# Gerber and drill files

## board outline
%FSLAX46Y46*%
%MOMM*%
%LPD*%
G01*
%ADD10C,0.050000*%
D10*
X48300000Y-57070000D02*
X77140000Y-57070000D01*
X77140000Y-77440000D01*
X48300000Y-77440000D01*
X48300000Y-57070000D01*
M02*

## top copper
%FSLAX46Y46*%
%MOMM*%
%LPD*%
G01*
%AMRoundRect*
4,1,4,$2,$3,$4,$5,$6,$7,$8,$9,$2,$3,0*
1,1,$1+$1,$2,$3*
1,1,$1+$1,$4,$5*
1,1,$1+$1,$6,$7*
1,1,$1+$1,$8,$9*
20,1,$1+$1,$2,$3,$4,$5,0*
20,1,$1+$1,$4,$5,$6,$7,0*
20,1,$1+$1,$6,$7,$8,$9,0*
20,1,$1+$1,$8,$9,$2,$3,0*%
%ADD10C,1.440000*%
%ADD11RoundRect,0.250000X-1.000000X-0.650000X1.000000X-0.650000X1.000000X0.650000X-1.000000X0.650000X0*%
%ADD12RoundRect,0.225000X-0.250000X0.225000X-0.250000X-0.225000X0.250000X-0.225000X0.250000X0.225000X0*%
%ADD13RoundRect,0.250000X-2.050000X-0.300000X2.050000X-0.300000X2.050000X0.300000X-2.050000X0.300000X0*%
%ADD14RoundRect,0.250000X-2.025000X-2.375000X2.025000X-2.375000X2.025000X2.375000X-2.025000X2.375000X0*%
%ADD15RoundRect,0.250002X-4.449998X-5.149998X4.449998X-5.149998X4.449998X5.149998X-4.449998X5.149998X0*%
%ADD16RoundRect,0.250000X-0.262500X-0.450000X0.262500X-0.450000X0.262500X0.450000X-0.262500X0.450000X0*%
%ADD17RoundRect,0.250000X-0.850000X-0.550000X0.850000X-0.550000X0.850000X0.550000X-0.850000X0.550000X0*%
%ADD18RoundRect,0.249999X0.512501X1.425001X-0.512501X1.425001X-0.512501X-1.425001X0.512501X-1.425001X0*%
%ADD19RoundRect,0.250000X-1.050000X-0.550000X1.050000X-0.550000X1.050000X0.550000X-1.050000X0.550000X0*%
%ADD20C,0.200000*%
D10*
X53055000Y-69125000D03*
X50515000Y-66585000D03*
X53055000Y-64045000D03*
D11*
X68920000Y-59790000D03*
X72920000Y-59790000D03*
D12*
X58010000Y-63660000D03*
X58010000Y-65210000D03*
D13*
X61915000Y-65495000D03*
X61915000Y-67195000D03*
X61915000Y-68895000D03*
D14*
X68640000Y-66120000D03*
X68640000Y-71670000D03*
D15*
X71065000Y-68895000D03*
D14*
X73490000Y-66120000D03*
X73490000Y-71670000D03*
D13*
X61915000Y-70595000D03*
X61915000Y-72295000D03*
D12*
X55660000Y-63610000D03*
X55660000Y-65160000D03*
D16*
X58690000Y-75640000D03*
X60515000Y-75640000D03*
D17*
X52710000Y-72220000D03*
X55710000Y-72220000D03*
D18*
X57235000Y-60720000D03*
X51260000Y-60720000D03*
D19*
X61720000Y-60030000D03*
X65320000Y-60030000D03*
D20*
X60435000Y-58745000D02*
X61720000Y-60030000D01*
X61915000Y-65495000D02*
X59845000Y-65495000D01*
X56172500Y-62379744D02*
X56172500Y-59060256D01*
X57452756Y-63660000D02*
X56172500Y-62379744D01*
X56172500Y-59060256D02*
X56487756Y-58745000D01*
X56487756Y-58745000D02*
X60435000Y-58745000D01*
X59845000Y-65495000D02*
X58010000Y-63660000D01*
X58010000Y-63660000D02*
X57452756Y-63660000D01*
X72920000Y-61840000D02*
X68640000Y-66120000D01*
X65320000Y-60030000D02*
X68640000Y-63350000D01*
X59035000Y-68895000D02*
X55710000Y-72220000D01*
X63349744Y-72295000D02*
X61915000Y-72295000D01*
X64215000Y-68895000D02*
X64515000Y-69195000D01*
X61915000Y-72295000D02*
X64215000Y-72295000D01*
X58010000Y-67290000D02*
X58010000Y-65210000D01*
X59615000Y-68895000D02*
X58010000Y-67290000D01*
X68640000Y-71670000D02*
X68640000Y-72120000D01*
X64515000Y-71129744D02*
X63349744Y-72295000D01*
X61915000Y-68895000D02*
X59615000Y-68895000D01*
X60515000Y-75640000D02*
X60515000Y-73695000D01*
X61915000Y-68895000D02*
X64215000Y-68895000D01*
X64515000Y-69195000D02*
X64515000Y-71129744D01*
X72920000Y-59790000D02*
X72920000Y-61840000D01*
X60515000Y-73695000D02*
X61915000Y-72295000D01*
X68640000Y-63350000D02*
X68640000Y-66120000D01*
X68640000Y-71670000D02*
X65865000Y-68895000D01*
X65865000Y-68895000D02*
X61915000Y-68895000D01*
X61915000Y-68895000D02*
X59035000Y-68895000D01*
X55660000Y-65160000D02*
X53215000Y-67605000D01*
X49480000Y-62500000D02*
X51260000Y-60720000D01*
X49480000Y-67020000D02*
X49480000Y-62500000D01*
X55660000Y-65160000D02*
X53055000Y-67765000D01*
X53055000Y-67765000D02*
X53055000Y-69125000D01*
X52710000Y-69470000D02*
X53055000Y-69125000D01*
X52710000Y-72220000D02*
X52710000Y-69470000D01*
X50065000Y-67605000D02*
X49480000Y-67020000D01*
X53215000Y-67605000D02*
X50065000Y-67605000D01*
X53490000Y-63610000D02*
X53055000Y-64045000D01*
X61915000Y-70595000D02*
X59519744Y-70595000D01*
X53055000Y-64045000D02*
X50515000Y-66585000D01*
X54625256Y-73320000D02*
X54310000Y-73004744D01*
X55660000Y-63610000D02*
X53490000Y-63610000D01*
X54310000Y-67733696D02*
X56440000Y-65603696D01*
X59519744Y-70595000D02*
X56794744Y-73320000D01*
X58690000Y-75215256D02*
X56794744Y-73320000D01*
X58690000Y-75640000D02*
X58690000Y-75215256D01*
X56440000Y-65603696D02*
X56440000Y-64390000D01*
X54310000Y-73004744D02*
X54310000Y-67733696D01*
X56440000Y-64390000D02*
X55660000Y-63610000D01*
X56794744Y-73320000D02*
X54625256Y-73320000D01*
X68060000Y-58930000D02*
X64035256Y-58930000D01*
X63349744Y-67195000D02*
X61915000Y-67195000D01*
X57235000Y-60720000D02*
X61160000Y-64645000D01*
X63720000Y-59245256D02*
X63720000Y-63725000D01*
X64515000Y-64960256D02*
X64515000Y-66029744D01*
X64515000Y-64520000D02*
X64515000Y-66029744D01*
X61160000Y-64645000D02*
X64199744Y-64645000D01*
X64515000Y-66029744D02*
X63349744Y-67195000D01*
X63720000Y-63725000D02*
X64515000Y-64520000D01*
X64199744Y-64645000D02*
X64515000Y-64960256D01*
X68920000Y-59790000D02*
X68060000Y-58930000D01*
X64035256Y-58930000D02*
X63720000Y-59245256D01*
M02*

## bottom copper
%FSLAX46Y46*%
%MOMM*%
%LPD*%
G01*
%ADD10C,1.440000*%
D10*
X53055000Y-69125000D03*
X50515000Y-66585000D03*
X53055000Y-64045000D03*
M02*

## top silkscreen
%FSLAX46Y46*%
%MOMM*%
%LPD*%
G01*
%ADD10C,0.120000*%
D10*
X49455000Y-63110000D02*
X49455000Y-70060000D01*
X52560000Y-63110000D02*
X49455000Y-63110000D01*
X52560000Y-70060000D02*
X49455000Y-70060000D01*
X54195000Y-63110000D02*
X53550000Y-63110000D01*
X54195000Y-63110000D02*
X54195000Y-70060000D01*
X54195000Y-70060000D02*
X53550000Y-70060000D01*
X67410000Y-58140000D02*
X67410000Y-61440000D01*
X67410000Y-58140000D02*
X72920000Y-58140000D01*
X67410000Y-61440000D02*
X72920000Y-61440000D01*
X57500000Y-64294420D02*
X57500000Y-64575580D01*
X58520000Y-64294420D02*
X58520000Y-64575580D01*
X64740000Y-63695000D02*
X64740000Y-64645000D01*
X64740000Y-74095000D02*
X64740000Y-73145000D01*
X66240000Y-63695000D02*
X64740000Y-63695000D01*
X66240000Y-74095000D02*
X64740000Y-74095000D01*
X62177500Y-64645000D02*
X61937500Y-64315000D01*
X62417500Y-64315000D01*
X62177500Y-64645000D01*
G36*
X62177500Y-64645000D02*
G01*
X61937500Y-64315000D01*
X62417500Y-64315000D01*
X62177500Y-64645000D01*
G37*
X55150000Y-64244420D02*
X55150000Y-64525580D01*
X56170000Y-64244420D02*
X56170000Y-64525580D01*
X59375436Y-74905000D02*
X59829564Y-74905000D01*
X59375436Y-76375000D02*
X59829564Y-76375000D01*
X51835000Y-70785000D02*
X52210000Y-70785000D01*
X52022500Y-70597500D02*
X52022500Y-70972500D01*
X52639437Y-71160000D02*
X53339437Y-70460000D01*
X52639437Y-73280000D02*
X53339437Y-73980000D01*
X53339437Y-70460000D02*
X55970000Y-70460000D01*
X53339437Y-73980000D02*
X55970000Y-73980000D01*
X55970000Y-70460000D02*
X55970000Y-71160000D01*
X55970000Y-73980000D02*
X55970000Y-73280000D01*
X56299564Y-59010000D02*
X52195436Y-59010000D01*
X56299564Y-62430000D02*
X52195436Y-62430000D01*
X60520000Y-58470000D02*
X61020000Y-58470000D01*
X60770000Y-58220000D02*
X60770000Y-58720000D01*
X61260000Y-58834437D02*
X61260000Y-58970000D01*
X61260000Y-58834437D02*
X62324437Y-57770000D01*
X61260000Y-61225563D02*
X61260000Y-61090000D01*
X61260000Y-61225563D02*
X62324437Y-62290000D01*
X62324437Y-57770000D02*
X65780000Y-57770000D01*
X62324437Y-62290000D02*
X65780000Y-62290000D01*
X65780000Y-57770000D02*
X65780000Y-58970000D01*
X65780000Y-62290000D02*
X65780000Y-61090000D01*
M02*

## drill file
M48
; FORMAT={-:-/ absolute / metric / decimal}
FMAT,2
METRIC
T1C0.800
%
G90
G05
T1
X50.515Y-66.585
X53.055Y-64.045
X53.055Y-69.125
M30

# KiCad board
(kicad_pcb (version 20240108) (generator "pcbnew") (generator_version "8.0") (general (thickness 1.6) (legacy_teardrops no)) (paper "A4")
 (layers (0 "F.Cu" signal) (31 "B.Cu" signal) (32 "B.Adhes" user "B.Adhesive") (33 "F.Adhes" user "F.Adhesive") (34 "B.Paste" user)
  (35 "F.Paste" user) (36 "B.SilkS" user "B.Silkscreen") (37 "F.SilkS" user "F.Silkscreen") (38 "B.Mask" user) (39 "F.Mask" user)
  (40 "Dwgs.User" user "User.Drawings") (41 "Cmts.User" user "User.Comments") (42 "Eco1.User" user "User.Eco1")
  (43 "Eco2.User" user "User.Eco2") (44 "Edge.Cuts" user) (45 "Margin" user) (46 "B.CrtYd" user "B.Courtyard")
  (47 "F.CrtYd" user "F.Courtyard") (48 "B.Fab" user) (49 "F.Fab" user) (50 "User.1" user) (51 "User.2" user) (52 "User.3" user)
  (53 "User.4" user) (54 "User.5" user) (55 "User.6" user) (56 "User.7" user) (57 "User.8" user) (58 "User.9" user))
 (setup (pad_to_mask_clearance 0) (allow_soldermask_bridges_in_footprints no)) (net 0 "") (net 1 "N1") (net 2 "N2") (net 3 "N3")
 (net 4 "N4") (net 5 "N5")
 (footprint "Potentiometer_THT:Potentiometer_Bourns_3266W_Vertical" (layer "F.Cu") (at 53.055 69.125 -90)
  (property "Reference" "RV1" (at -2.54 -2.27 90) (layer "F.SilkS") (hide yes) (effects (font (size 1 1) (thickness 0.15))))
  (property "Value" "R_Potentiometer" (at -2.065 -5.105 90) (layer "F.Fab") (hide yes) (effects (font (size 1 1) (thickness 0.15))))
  (fp_line (start -6.015 3.6) (end 0.935 3.6) (stroke (width 0.12) (type solid)) (layer "F.SilkS"))
  (fp_line (start -6.015 0.495) (end -6.015 3.6) (stroke (width 0.12) (type solid)) (layer "F.SilkS"))
  (fp_line (start 0.935 0.495) (end 0.935 3.6) (stroke (width 0.12) (type solid)) (layer "F.SilkS"))
  (fp_line (start -6.015 -1.14) (end -6.015 -0.495) (stroke (width 0.12) (type solid)) (layer "F.SilkS"))
  (fp_line (start -6.015 -1.14) (end 0.935 -1.14) (stroke (width 0.12) (type solid)) (layer "F.SilkS"))
  (fp_line (start 0.935 -1.14) (end 0.935 -0.495) (stroke (width 0.12) (type solid)) (layer "F.SilkS"))
  (pad "1" thru_hole circle (at 0 0 270) (size 1.44 1.44) (drill 0.8) (layers "*.Cu" "*.Mask") (remove_unused_layers no) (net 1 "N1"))
  (pad "2" thru_hole circle (at -2.54 2.54 270) (size 1.44 1.44) (drill 0.8) (layers "*.Cu" "*.Mask") (remove_unused_layers no) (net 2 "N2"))
  (pad "3" thru_hole circle (at -5.08 0 270) (size 1.44 1.44) (drill 0.8) (layers "*.Cu" "*.Mask") (remove_unused_layers no) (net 2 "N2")))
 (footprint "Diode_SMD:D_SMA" (layer "F.Cu") (at 70.92 59.79)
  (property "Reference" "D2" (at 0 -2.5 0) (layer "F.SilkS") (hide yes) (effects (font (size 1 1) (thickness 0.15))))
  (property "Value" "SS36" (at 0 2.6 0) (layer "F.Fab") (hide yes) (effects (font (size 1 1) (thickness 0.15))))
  (fp_line (start -3.51 -1.65) (end -3.51 1.65) (stroke (width 0.12) (type solid)) (layer "F.SilkS"))
  (fp_line (start -3.51 -1.65) (end 2 -1.65) (stroke (width 0.12) (type solid)) (layer "F.SilkS"))
  (fp_line (start -3.51 1.65) (end 2 1.65) (stroke (width 0.12) (type solid)) (layer "F.SilkS"))
  (pad "1" smd roundrect (at -2 0) (size 2.5 1.8) (layers "F.Cu" "F.Paste" "F.Mask") (roundrect_rratio 0.1388888889) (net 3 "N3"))
  (pad "2" smd roundrect (at 2 0) (size 2.5 1.8) (layers "F.Cu" "F.Paste" "F.Mask") (roundrect_rratio 0.1388888889) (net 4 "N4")))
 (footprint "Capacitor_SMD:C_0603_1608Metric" (layer "F.Cu") (at 58.01 64.435 -90)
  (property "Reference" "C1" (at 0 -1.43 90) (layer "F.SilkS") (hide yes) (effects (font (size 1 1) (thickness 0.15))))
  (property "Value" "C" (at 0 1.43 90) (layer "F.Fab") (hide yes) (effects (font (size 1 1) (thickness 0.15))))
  (fp_line (start -0.14058 0.51) (end 0.14058 0.51) (stroke (width 0.12) (type solid)) (layer "F.SilkS"))
  (fp_line (start -0.14058 -0.51) (end 0.14058 -0.51) (stroke (width 0.12) (type solid)) (layer "F.SilkS"))
  (pad "1" smd roundrect (at -0.775 0 270) (size 0.9 0.95) (layers "F.Cu" "F.Paste" "F.Mask") (roundrect_rratio 0.25) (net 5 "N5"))
  (pad "2" smd roundrect (at 0.775 0 270) (size 0.9 0.95) (layers "F.Cu" "F.Paste" "F.Mask") (roundrect_rratio 0.25) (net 4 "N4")))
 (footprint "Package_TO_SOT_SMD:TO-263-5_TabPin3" (layer "F.Cu") (at 69.565 68.895)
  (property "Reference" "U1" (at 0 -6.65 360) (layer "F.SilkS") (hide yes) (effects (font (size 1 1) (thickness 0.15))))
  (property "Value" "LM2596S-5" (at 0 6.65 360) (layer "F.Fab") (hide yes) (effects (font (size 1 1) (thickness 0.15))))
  (fp_line (start -4.825 -5.2) (end -4.825 -4.25) (stroke (width 0.12) (type solid)) (layer "F.SilkS"))
  (fp_line (start -4.825 5.2) (end -4.825 4.25) (stroke (width 0.12) (type solid)) (layer "F.SilkS"))
  (fp_line (start -3.325 -5.2) (end -4.825 -5.2) (stroke (width 0.12) (type solid)) (layer "F.SilkS"))
  (fp_line (start -3.325 5.2) (end -4.825 5.2) (stroke (width 0.12) (type solid)) (layer "F.SilkS"))
  (fp_poly
   (pts (xy -7.3875 -4.25) (xy -7.6275 -4.58) (xy -7.1475 -4.58) (xy -7.3875 -4.25)) (stroke (width 0.12) (type solid)) (fill solid)
   (layer "F.SilkS"))
  (pad "1" smd roundrect (at -7.65 -3.4) (size 4.6 1.1) (layers "F.Cu" "F.Paste" "F.Mask") (roundrect_rratio 0.227273) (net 5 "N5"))
  (pad "2" smd roundrect (at -7.65 -1.7) (size 4.6 1.1) (layers "F.Cu" "F.Paste" "F.Mask") (roundrect_rratio 0.227273) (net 3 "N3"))
  (pad "3" smd roundrect (at -7.65 0) (size 4.6 1.1) (layers "F.Cu" "F.Paste" "F.Mask") (roundrect_rratio 0.227273) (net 4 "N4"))
  (pad "3" smd roundrect (at -0.925 -2.775) (size 4.55 5.25) (layers "F.Cu" "F.Paste") (roundrect_rratio 0.054945) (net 4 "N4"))
  (pad "3" smd roundrect (at -0.925 2.775) (size 4.55 5.25) (layers "F.Cu" "F.Paste") (roundrect_rratio 0.054945) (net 4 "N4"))
  (pad "3" smd roundrect (at 1.5 0) (size 9.4 10.8) (layers "F.Cu" "F.Mask") (roundrect_rratio 0.026596) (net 4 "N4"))
  (pad "3" smd roundrect (at 3.925 -2.775) (size 4.55 5.25) (layers "F.Cu" "F.Paste") (roundrect_rratio 0.054945) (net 4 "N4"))
  (pad "3" smd roundrect (at 3.925 2.775) (size 4.55 5.25) (layers "F.Cu" "F.Paste") (roundrect_rratio 0.054945) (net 4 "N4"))
  (pad "4" smd roundrect (at -7.65 1.7) (size 4.6 1.1) (layers "F.Cu" "F.Paste" "F.Mask") (roundrect_rratio 0.227273) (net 2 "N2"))
  (pad "5" smd roundrect (at -7.65 3.4) (size 4.6 1.1) (layers "F.Cu" "F.Paste" "F.Mask") (roundrect_rratio 0.227273) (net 4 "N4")))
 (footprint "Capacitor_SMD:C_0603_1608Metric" (layer "F.Cu") (at 55.66 64.385 -90)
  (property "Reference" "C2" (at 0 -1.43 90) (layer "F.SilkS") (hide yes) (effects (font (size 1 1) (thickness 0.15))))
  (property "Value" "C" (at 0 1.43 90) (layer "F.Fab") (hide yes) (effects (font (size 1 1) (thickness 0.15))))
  (fp_line (start -0.14058 0.51) (end 0.14058 0.51) (stroke (width 0.12) (type solid)) (layer "F.SilkS"))
  (fp_line (start -0.14058 -0.51) (end 0.14058 -0.51) (stroke (width 0.12) (type solid)) (layer "F.SilkS"))
  (pad "1" smd roundrect (at -0.775 0 270) (size 0.9 0.95) (layers "F.Cu" "F.Paste" "F.Mask") (roundrect_rratio 0.25) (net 2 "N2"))
  (pad "2" smd roundrect (at 0.775 0 270) (size 0.9 0.95) (layers "F.Cu" "F.Paste" "F.Mask") (roundrect_rratio 0.25) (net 1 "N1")))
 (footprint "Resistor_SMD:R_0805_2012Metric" (layer "F.Cu") (at 59.6025 75.64)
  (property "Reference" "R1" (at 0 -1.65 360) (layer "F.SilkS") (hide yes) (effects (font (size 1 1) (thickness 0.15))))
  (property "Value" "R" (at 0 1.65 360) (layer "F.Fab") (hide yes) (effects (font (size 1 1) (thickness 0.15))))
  (fp_line (start -0.227064 -0.735) (end 0.227064 -0.735) (stroke (width 0.12) (type solid)) (layer "F.SilkS"))
  (fp_line (start -0.227064 0.735) (end 0.227064 0.735) (stroke (width 0.12) (type solid)) (layer "F.SilkS"))
  (pad "1" smd roundrect (at -0.9125 0) (size 1.025 1.4) (layers "F.Cu" "F.Paste" "F.Mask") (roundrect_rratio 0.243902) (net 2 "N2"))
  (pad "2" smd roundrect (at 0.9125 0) (size 1.025 1.4) (layers "F.Cu" "F.Paste" "F.Mask") (roundrect_rratio 0.243902) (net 4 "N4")))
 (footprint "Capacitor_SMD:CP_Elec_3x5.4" (layer "F.Cu") (at 54.21 72.22)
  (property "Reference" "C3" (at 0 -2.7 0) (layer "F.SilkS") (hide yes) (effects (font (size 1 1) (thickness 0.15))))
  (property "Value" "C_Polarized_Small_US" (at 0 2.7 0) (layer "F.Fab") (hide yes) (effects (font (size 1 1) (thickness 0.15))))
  (fp_line (start -2.375 -1.435) (end -2 -1.435) (stroke (width 0.12) (type solid)) (layer "F.SilkS"))
  (fp_line (start -2.1875 -1.6225) (end -2.1875 -1.2475) (stroke (width 0.12) (type solid)) (layer "F.SilkS"))
  (fp_line (start -1.570563 -1.06) (end -0.870563 -1.76) (stroke (width 0.12) (type solid)) (layer "F.SilkS"))
  (fp_line (start -1.570563 1.06) (end -0.870563 1.76) (stroke (width 0.12) (type solid)) (layer "F.SilkS"))
  (fp_line (start -0.870563 -1.76) (end 1.76 -1.76) (stroke (width 0.12) (type solid)) (layer "F.SilkS"))
  (fp_line (start -0.870563 1.76) (end 1.76 1.76) (stroke (width 0.12) (type solid)) (layer "F.SilkS"))
  (fp_line (start 1.76 -1.76) (end 1.76 -1.06) (stroke (width 0.12) (type solid)) (layer "F.SilkS"))
  (fp_line (start 1.76 1.76) (end 1.76 1.06) (stroke (width 0.12) (type solid)) (layer "F.SilkS"))
  (pad "1" smd roundrect (at -1.5 0) (size 2.2 1.6) (layers "F.Cu" "F.Paste" "F.Mask") (roundrect_rratio 0.15625) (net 1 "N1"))
  (pad "2" smd roundrect (at 1.5 0) (size 2.2 1.6) (layers "F.Cu" "F.Paste" "F.Mask") (roundrect_rratio 0.15625) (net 4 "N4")))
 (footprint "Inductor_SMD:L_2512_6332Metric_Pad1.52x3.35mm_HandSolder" (layer "F.Cu") (at 54.2475 60.72 180)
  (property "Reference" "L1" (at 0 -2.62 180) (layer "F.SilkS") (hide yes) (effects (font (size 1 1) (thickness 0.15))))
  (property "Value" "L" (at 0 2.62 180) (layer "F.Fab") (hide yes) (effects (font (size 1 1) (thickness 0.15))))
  (fp_line (start -2.052064 1.71) (end 2.052064 1.71) (stroke (width 0.12) (type solid)) (layer "F.SilkS"))
  (fp_line (start -2.052064 -1.71) (end 2.052064 -1.71) (stroke (width 0.12) (type solid)) (layer "F.SilkS"))
  (pad "1" smd roundrect (at -2.9875 0 180) (size 1.525 3.35) (layers "F.Cu" "F.Paste" "F.Mask") (roundrect_rratio 0.163934) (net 3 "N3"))
  (pad "2" smd roundrect (at 2.9875 0 180) (size 1.525 3.35) (layers "F.Cu" "F.Paste" "F.Mask") (roundrect_rratio 0.163934) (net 1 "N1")))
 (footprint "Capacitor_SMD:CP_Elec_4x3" (layer "F.Cu") (at 63.52 60.03)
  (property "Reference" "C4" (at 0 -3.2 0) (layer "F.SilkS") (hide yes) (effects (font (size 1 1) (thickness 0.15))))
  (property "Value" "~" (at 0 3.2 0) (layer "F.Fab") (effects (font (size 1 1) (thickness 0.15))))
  (fp_line (start -3 -1.56) (end -2.5 -1.56) (stroke (width 0.12) (type solid)) (layer "F.SilkS"))
  (fp_line (start -2.75 -1.81) (end -2.75 -1.31) (stroke (width 0.12) (type solid)) (layer "F.SilkS"))
  (fp_line (start -2.26 -1.195563) (end -2.26 -1.06) (stroke (width 0.12) (type solid)) (layer "F.SilkS"))
  (fp_line (start -2.26 -1.195563) (end -1.195563 -2.26) (stroke (width 0.12) (type solid)) (layer "F.SilkS"))
  (fp_line (start -2.26 1.195563) (end -2.26 1.06) (stroke (width 0.12) (type solid)) (layer "F.SilkS"))
  (fp_line (start -2.26 1.195563) (end -1.195563 2.26) (stroke (width 0.12) (type solid)) (layer "F.SilkS"))
  (fp_line (start -1.195563 -2.26) (end 2.26 -2.26) (stroke (width 0.12) (type solid)) (layer "F.SilkS"))
  (fp_line (start -1.195563 2.26) (end 2.26 2.26) (stroke (width 0.12) (type solid)) (layer "F.SilkS"))
  (fp_line (start 2.26 -2.26) (end 2.26 -1.06) (stroke (width 0.12) (type solid)) (layer "F.SilkS"))
  (fp_line (start 2.26 2.26) (end 2.26 1.06) (stroke (width 0.12) (type solid)) (layer "F.SilkS"))
  (pad "1" smd roundrect (at -1.8 0) (size 2.6 1.6) (layers "F.Cu" "F.Paste" "F.Mask") (roundrect_rratio 0.15625) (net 5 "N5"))
  (pad "2" smd roundrect (at 1.8 0) (size 2.6 1.6) (layers "F.Cu" "F.Paste" "F.Mask") (roundrect_rratio 0.15625) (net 4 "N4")))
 (gr_rect (start 48.3 57.07) (end 77.14 77.44) (stroke (width 0.05) (type default)) (fill none) (layer "Edge.Cuts"))
 (segment (start 60.435 58.745) (end 61.72 60.03) (width 0.2) (layer "F.Cu") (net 5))
 (segment (start 61.915 65.495) (end 59.845 65.495) (width 0.2) (layer "F.Cu") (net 5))
 (segment (start 56.1725 62.379744) (end 56.1725 59.060256) (width 0.2) (layer "F.Cu") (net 5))
 (segment (start 57.452756 63.66) (end 56.1725 62.379744) (width 0.2) (layer "F.Cu") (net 5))
 (segment (start 56.1725 59.060256) (end 56.487756 58.745) (width 0.2) (layer "F.Cu") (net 5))
 (segment (start 56.487756 58.745) (end 60.435 58.745) (width 0.2) (layer "F.Cu") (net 5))
 (segment (start 59.845 65.495) (end 58.01 63.66) (width 0.2) (layer "F.Cu") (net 5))
 (segment (start 58.01 63.66) (end 57.452756 63.66) (width 0.2) (layer "F.Cu") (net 5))
 (segment (start 72.92 61.84) (end 68.64 66.12) (width 0.2) (layer "F.Cu") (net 4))
 (segment (start 65.32 60.03) (end 68.64 63.35) (width 0.2) (layer "F.Cu") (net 4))
 (segment (start 59.035 68.895) (end 55.71 72.22) (width 0.2) (layer "F.Cu") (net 4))
 (segment (start 63.349744 72.295) (end 61.915 72.295) (width 0.2) (layer "F.Cu") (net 4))
 (segment (start 64.215 68.895) (end 64.515 69.195) (width 0.2) (layer "F.Cu") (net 4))
 (segment (start 61.915 72.295) (end 64.215 72.295) (width 0.2) (layer "F.Cu") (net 4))
 (segment (start 58.01 67.29) (end 58.01 65.21) (width 0.2) (layer "F.Cu") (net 4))
 (segment (start 59.615 68.895) (end 58.01 67.29) (width 0.2) (layer "F.Cu") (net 4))
 (segment (start 68.64 71.67) (end 68.64 72.12) (width 0.2) (layer "F.Cu") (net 4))
 (segment (start 64.515 71.129744) (end 63.349744 72.295) (width 0.2) (layer "F.Cu") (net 4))
 (segment (start 61.915 68.895) (end 59.615 68.895) (width 0.2) (layer "F.Cu") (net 4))
 (segment (start 60.515 75.64) (end 60.515 73.695) (width 0.2) (layer "F.Cu") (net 4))
 (segment (start 61.915 68.895) (end 64.215 68.895) (width 0.2) (layer "F.Cu") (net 4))
 (segment (start 64.515 69.195) (end 64.515 71.129744) (width 0.2) (layer "F.Cu") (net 4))
 (segment (start 72.92 59.79) (end 72.92 61.84) (width 0.2) (layer "F.Cu") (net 4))
 (segment (start 60.515 73.695) (end 61.915 72.295) (width 0.2) (layer "F.Cu") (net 4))
 (segment (start 68.64 63.35) (end 68.64 66.12) (width 0.2) (layer "F.Cu") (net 4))
 (segment (start 68.64 71.67) (end 65.865 68.895) (width 0.2) (layer "F.Cu") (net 4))
 (segment (start 65.865 68.895) (end 61.915 68.895) (width 0.2) (layer "F.Cu") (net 4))
 (segment (start 61.915 68.895) (end 59.035 68.895) (width 0.2) (layer "F.Cu") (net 4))
 (segment (start 55.66 65.16) (end 53.215 67.605) (width 0.2) (layer "F.Cu") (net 1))
 (segment (start 49.48 62.5) (end 51.26 60.72) (width 0.2) (layer "F.Cu") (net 1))
 (segment (start 49.48 67.02) (end 49.48 62.5) (width 0.2) (layer "F.Cu") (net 1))
 (segment (start 55.66 65.16) (end 53.055 67.765) (width 0.2) (layer "F.Cu") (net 1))
 (segment (start 53.055 67.765) (end 53.055 69.125) (width 0.2) (layer "F.Cu") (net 1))
 (segment (start 52.71 69.47) (end 53.055 69.125) (width 0.2) (layer "F.Cu") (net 1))
 (segment (start 52.71 72.22) (end 52.71 69.47) (width 0.2) (layer "F.Cu") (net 1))
 (segment (start 50.065 67.605) (end 49.48 67.02) (width 0.2) (layer "F.Cu") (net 1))
 (segment (start 53.215 67.605) (end 50.065 67.605) (width 0.2) (layer "F.Cu") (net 1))
 (segment (start 53.49 63.61) (end 53.055 64.045) (width 0.2) (layer "F.Cu") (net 2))
 (segment (start 61.915 70.595) (end 59.519744 70.595) (width 0.2) (layer "F.Cu") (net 2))
 (segment (start 53.055 64.045) (end 50.515 66.585) (width 0.2) (layer "F.Cu") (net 2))
 (segment (start 54.625256 73.32) (end 54.31 73.004744) (width 0.2) (layer "F.Cu") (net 2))
 (segment (start 55.66 63.61) (end 53.49 63.61) (width 0.2) (layer "F.Cu") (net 2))
 (segment (start 54.31 67.733696) (end 56.44 65.603696) (width 0.2) (layer "F.Cu") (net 2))
 (segment (start 59.519744 70.595) (end 56.794744 73.32) (width 0.2) (layer "F.Cu") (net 2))
 (segment (start 58.69 75.215256) (end 56.794744 73.32) (width 0.2) (layer "F.Cu") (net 2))
 (segment (start 58.69 75.64) (end 58.69 75.215256) (width 0.2) (layer "F.Cu") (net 2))
 (segment (start 56.44 65.603696) (end 56.44 64.39) (width 0.2) (layer "F.Cu") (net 2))
 (segment (start 54.31 73.004744) (end 54.31 67.733696) (width 0.2) (layer "F.Cu") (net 2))
 (segment (start 56.44 64.39) (end 55.66 63.61) (width 0.2) (layer "F.Cu") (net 2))
 (segment (start 56.794744 73.32) (end 54.625256 73.32) (width 0.2) (layer "F.Cu") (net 2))
 (segment (start 68.06 58.93) (end 64.035256 58.93) (width 0.2) (layer "F.Cu") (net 3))
 (segment (start 63.349744 67.195) (end 61.915 67.195) (width 0.2) (layer "F.Cu") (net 3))
 (segment (start 57.235 60.72) (end 61.16 64.645) (width 0.2) (layer "F.Cu") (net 3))
 (segment (start 63.72 59.245256) (end 63.72 63.725) (width 0.2) (layer "F.Cu") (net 3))
 (segment (start 64.515 64.960256) (end 64.515 66.029744) (width 0.2) (layer "F.Cu") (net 3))
 (segment (start 64.515 64.52) (end 64.515 66.029744) (width 0.2) (layer "F.Cu") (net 3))
 (segment (start 61.16 64.645) (end 64.199744 64.645) (width 0.2) (layer "F.Cu") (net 3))
 (segment (start 64.515 66.029744) (end 63.349744 67.195) (width 0.2) (layer "F.Cu") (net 3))
 (segment (start 63.72 63.725) (end 64.515 64.52) (width 0.2) (layer "F.Cu") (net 3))
 (segment (start 64.199744 64.645) (end 64.515 64.960256) (width 0.2) (layer "F.Cu") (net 3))
 (segment (start 68.92 59.79) (end 68.06 58.93) (width 0.2) (layer "F.Cu") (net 3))
 (segment (start 64.035256 58.93) (end 63.72 59.245256) (width 0.2) (layer "F.Cu") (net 3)))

